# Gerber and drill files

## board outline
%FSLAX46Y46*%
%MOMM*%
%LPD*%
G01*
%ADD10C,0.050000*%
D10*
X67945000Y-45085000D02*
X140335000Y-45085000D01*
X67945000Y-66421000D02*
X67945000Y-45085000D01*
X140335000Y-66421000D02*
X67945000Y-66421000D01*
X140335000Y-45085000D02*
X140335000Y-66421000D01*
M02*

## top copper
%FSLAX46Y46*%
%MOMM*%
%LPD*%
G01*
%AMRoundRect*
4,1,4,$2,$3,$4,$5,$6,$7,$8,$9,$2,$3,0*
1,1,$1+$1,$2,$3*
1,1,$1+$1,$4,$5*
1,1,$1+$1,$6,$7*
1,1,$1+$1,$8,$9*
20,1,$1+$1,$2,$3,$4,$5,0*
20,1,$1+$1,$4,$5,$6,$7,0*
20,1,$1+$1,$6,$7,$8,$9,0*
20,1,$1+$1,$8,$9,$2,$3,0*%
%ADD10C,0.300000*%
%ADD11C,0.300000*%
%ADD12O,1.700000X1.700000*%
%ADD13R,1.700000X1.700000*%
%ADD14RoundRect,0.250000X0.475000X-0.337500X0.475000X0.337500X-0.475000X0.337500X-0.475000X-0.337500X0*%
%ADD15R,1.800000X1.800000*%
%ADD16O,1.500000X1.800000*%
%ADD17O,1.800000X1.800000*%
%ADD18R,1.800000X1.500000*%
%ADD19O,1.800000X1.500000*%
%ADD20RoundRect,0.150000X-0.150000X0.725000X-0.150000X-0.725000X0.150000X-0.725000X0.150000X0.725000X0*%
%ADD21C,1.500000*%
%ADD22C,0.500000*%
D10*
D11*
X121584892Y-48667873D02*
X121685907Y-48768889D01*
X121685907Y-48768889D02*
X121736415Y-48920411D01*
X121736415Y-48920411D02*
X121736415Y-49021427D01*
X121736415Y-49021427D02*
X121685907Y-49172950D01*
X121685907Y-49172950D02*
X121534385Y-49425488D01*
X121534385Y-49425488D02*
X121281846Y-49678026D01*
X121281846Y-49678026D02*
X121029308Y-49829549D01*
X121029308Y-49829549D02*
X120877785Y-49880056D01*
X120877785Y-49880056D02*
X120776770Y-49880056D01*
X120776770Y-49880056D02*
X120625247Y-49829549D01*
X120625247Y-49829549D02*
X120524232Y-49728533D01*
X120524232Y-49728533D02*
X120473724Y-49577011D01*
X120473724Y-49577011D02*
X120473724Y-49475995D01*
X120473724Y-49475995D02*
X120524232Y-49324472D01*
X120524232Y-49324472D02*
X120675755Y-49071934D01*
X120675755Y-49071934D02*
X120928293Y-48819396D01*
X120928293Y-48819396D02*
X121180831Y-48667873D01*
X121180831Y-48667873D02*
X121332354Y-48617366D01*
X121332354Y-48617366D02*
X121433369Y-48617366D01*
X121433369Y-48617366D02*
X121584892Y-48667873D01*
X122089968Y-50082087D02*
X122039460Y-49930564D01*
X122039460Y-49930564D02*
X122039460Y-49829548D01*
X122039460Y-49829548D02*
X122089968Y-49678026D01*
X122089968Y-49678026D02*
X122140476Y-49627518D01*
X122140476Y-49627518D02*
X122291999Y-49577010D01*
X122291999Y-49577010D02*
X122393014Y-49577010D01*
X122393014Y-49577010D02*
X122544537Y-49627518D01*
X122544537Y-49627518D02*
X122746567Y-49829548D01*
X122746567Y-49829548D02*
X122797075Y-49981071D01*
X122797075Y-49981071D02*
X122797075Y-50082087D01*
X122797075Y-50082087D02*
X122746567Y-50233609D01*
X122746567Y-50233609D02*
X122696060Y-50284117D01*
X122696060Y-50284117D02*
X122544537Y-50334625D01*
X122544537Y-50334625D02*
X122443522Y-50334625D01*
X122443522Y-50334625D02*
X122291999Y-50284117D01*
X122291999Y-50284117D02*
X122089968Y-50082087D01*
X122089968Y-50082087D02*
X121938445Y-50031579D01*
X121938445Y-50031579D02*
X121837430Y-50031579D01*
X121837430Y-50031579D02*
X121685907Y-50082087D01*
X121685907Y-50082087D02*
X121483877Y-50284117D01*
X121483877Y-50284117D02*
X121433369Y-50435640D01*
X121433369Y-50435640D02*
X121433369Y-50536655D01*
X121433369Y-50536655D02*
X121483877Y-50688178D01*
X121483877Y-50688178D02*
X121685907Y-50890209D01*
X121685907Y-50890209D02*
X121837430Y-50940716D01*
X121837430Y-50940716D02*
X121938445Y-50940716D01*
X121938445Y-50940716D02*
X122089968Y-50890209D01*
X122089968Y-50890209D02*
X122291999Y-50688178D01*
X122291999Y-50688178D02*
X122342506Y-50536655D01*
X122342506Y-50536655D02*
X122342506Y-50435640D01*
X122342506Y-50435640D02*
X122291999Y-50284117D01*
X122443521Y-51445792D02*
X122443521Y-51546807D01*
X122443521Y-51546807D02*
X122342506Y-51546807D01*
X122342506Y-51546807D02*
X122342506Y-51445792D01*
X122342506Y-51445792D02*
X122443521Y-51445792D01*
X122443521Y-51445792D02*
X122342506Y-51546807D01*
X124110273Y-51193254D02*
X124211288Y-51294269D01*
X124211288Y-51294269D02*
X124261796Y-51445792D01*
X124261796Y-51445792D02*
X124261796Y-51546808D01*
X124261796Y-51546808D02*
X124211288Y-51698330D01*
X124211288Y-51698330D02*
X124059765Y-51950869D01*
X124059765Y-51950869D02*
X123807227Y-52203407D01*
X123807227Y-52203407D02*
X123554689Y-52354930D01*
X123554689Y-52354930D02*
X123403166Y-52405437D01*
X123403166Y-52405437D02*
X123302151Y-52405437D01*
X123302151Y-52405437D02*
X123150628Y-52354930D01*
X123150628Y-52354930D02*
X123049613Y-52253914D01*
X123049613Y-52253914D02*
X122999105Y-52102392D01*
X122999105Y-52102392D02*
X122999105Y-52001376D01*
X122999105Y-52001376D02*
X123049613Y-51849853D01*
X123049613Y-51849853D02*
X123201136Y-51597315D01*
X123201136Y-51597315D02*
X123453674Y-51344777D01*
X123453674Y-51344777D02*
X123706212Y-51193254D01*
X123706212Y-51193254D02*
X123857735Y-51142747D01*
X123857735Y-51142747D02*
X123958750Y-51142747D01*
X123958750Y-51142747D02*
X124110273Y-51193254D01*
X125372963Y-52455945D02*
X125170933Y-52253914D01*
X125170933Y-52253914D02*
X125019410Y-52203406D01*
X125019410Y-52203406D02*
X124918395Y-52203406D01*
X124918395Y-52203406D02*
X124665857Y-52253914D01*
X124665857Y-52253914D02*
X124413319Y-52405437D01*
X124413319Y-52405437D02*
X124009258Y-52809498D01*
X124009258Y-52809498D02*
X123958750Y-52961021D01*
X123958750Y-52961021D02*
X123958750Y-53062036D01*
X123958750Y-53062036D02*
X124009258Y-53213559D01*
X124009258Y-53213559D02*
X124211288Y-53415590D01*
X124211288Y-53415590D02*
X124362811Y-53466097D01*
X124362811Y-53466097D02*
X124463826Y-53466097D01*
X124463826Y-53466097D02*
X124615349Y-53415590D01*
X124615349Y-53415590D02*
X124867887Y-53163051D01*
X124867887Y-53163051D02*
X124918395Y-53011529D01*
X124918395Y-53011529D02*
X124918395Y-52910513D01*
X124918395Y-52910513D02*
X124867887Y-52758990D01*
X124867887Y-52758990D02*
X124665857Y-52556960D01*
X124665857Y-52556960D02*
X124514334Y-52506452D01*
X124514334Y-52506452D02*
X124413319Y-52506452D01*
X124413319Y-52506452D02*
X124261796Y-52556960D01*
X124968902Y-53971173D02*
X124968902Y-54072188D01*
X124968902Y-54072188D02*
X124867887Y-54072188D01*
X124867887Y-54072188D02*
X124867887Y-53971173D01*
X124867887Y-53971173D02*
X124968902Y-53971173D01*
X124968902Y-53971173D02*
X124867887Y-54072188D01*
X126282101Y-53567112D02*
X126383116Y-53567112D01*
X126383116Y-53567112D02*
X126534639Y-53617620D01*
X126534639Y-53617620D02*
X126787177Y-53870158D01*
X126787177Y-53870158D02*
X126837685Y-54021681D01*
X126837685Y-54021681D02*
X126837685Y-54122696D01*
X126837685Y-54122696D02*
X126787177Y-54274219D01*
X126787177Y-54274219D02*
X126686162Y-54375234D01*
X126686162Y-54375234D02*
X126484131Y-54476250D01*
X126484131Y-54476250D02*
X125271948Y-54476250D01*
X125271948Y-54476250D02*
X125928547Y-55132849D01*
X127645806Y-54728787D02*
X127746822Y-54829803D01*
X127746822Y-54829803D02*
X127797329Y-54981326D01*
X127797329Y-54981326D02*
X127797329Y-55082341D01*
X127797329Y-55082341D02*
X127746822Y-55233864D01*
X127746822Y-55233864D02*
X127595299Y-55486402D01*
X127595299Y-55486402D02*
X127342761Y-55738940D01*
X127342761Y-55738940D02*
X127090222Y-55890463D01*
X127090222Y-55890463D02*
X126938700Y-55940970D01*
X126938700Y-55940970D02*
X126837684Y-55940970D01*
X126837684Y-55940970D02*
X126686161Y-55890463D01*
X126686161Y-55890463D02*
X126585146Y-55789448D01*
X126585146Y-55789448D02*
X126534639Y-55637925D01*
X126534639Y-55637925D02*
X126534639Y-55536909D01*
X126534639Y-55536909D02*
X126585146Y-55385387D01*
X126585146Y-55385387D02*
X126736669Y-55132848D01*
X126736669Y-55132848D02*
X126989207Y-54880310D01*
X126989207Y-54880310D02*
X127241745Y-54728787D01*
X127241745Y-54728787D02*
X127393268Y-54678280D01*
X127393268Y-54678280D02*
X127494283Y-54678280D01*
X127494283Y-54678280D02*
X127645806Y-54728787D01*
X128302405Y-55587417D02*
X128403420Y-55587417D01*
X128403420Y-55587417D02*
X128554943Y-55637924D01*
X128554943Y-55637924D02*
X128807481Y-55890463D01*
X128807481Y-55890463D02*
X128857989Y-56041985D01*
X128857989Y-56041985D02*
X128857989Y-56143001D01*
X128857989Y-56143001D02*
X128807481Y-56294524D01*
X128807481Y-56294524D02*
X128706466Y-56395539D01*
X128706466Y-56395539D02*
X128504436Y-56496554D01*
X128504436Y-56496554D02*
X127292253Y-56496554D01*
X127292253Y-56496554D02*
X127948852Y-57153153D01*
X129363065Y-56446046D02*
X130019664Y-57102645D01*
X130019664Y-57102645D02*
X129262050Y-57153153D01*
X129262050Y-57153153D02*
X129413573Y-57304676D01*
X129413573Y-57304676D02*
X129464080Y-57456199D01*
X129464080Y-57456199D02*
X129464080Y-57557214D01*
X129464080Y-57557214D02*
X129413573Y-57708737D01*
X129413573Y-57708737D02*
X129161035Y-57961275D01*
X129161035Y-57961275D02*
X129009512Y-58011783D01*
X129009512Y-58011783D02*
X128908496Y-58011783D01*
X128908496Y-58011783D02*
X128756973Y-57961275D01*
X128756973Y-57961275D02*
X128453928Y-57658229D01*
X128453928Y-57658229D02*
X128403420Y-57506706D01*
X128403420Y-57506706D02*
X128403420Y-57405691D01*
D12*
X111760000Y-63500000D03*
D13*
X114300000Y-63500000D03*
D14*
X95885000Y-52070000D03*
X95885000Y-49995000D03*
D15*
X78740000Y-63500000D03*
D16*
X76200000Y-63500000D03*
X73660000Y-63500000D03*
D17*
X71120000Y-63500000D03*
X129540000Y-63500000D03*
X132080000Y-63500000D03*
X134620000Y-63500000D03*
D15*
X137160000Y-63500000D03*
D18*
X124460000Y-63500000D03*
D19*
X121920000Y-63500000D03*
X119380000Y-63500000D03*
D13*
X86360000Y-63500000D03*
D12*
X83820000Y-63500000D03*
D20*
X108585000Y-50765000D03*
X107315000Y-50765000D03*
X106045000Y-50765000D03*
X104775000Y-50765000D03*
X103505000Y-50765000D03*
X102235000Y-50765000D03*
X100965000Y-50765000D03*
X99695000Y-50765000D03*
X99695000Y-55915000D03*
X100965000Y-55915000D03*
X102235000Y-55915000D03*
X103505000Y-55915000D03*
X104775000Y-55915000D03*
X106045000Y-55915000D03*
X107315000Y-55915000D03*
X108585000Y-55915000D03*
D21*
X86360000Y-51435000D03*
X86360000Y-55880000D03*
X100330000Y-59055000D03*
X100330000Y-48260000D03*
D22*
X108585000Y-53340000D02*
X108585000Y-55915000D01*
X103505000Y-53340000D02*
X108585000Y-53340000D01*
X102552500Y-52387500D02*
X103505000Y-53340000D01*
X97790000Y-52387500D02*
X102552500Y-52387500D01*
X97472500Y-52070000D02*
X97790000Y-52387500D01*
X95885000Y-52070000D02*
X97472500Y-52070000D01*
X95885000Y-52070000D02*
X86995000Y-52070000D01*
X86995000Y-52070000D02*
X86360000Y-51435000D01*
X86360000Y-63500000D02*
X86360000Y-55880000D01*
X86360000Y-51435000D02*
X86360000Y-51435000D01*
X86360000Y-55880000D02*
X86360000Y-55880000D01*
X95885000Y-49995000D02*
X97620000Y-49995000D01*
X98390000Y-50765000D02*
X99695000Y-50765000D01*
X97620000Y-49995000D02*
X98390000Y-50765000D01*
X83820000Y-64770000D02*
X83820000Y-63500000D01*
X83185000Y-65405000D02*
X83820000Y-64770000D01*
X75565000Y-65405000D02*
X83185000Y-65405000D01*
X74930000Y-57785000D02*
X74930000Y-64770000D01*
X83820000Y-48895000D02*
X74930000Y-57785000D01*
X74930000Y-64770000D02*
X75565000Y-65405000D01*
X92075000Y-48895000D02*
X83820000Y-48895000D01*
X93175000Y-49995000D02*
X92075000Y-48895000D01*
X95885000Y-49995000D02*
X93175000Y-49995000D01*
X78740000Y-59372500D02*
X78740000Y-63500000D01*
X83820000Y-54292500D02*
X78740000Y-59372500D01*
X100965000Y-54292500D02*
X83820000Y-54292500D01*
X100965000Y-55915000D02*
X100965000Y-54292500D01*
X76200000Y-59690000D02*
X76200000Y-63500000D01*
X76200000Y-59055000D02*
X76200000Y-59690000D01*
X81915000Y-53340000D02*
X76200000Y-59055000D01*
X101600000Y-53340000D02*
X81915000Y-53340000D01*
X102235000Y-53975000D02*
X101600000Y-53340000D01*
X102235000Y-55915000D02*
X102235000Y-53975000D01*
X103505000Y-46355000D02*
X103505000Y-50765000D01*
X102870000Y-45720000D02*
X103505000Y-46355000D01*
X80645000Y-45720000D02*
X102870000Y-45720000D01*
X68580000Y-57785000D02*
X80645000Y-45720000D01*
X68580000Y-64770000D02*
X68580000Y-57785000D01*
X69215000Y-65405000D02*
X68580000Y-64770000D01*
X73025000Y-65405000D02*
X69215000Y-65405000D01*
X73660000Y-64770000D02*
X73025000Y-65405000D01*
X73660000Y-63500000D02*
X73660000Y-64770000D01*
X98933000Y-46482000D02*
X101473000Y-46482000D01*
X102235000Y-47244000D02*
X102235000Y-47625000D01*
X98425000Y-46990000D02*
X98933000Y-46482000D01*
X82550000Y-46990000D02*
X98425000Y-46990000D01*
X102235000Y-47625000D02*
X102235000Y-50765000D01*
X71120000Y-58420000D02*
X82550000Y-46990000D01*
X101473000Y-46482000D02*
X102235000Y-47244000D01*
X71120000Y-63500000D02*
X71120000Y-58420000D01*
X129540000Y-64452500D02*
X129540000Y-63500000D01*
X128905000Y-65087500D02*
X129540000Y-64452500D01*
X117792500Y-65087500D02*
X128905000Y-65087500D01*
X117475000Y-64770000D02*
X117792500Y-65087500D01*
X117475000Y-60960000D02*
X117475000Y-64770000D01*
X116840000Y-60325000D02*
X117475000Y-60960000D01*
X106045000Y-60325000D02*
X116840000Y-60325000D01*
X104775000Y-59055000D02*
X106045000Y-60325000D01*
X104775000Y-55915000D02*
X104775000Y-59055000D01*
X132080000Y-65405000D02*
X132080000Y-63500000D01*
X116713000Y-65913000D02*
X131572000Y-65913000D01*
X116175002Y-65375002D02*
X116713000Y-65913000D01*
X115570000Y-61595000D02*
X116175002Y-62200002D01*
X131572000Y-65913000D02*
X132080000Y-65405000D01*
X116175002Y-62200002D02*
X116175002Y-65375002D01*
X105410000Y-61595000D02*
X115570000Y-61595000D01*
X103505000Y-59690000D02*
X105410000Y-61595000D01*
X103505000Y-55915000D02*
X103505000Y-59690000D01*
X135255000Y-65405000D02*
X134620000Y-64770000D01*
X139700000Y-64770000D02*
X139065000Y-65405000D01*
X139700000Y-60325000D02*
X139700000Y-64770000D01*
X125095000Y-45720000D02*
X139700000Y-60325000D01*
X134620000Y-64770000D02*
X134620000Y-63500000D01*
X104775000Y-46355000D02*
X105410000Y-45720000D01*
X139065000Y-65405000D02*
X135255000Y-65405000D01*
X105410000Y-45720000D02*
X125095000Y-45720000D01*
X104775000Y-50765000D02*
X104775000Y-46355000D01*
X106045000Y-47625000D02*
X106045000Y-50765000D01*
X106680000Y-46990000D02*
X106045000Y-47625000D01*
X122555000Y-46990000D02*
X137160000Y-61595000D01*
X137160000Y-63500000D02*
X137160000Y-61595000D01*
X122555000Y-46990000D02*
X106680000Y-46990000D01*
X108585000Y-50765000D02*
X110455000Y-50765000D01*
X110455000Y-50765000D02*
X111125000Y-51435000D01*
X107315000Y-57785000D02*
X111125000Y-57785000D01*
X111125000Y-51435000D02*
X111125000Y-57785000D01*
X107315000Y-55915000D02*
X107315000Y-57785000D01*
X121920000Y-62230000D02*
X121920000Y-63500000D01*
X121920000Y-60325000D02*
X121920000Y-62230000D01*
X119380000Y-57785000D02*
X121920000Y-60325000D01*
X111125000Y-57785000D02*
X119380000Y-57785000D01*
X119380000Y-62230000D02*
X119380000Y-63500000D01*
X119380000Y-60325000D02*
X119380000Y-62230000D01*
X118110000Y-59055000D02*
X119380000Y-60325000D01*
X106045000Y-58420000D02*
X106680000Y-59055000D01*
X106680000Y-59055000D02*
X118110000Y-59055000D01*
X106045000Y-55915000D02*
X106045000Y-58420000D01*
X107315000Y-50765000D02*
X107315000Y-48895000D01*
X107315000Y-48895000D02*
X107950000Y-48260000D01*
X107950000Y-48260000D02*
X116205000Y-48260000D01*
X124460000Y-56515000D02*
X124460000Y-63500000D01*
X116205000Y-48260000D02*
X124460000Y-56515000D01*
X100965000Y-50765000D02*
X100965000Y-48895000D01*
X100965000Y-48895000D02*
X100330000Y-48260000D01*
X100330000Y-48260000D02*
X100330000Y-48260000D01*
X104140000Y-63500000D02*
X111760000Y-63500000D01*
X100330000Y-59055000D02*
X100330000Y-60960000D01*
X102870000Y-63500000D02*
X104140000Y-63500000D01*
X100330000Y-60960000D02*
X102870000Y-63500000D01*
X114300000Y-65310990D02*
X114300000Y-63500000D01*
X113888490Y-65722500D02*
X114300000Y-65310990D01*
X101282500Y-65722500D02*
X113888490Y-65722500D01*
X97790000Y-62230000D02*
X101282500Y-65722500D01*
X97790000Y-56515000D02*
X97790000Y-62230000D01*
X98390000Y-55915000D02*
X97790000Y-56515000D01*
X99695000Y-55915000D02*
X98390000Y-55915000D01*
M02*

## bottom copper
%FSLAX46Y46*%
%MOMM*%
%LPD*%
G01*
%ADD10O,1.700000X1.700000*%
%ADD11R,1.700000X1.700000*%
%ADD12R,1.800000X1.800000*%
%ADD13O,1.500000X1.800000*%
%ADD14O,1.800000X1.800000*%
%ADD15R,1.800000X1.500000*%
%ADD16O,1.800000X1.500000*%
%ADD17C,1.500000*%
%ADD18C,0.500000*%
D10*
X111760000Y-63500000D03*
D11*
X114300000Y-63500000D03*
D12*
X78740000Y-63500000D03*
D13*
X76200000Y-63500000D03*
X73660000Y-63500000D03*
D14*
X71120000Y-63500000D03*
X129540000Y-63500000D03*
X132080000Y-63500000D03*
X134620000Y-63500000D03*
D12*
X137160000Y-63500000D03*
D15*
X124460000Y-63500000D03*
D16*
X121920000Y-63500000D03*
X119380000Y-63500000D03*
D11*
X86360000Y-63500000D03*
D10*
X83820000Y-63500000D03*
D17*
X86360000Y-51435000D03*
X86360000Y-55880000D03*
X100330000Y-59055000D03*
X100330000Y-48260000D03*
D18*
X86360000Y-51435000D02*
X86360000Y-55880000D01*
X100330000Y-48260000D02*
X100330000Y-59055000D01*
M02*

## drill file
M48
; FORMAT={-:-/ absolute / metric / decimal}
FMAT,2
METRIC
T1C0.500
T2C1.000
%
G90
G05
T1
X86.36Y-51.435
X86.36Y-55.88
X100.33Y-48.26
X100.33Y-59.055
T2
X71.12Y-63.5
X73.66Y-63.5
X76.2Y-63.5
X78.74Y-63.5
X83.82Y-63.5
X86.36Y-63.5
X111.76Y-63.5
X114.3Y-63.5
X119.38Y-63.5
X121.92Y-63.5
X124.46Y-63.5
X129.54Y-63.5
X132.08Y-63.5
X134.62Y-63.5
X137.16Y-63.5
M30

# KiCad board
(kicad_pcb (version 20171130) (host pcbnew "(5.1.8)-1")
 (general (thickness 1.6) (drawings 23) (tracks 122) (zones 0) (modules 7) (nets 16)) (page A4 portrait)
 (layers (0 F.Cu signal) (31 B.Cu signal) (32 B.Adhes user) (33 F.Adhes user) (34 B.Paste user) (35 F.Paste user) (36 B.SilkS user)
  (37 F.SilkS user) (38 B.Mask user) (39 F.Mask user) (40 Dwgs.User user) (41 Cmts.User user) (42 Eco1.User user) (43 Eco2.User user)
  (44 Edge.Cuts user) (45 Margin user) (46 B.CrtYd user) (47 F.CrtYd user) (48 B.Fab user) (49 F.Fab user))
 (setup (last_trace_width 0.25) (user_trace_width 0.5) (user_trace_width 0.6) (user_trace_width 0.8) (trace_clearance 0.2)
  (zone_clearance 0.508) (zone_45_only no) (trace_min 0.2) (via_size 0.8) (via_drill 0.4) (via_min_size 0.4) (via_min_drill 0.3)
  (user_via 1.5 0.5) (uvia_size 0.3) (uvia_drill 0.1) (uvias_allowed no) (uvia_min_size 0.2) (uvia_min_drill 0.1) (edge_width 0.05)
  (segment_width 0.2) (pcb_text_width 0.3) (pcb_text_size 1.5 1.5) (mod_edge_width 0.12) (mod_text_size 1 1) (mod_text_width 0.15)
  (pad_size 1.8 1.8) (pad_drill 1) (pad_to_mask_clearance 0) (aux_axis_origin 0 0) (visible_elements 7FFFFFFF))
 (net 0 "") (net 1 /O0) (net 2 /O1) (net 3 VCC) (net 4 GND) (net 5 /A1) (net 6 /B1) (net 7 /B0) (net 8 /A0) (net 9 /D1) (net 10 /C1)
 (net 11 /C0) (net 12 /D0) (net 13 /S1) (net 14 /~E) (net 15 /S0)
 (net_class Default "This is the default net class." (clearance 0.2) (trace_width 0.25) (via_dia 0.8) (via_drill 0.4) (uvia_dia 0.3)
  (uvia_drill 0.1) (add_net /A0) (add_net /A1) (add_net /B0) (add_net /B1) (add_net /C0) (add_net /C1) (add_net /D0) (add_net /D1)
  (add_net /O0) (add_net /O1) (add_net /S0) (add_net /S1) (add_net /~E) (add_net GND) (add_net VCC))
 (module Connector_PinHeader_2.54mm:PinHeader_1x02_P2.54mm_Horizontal (layer F.Cu) (at 114.3 63.5 270)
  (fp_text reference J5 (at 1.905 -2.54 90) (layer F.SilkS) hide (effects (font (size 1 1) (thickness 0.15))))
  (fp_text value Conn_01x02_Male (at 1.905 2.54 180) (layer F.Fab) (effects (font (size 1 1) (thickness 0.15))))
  (pad 2 thru_hole oval (at 0 2.54 270) (size 1.7 1.7) (drill 1) (layers *.Cu *.Mask) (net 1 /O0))
  (pad 1 thru_hole rect (at 0 0 270) (size 1.7 1.7) (drill 1) (layers *.Cu *.Mask) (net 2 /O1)))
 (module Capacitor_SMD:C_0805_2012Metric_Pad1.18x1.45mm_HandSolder (layer F.Cu) (at 95.885 51.0325 90)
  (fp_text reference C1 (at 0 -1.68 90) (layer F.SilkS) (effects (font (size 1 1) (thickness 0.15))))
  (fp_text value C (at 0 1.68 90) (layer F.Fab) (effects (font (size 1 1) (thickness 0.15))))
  (pad 1 smd roundrect (at -1.0375 0 90) (size 1.175 1.45) (layers F.Cu F.Paste F.Mask) (roundrect_rratio 0.2127659574468085) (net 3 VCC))
  (pad 2 smd roundrect (at 1.0375 0 90) (size 1.175 1.45) (layers F.Cu F.Paste F.Mask) (roundrect_rratio 0.2127659574468085) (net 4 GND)))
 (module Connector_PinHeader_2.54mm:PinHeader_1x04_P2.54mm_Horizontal (layer F.Cu) (at 78.74 63.5 270)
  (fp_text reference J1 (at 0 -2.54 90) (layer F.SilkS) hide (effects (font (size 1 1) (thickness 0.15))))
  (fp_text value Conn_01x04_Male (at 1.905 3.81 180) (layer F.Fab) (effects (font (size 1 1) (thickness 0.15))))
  (pad 1 thru_hole rect (at 0 0 270) (size 1.8 1.8) (drill 1) (layers *.Cu *.Mask) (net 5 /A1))
  (pad 2 thru_hole oval (at 0 2.54 270) (size 1.8 1.5) (drill 1) (layers *.Cu *.Mask) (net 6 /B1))
  (pad 3 thru_hole oval (at 0 5.08 270) (size 1.8 1.5) (drill 1) (layers *.Cu *.Mask) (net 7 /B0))
  (pad 4 thru_hole oval (at 0 7.62 270) (size 1.8 1.8) (drill 1) (layers *.Cu *.Mask) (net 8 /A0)))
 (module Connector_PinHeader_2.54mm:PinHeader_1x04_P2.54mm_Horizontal (layer F.Cu) (at 137.16 63.5 270)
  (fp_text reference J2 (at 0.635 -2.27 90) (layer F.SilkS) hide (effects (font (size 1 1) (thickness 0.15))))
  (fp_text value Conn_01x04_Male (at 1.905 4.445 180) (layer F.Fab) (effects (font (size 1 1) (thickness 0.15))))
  (pad 4 thru_hole oval (at 0 7.62 270) (size 1.8 1.8) (drill 1) (layers *.Cu *.Mask) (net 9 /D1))
  (pad 3 thru_hole oval (at 0 5.08 270) (size 1.8 1.8) (drill 1) (layers *.Cu *.Mask) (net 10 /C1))
  (pad 2 thru_hole oval (at 0 2.54 270) (size 1.8 1.8) (drill 1) (layers *.Cu *.Mask) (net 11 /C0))
  (pad 1 thru_hole rect (at 0 0 270) (size 1.8 1.8) (drill 1) (layers *.Cu *.Mask) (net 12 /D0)))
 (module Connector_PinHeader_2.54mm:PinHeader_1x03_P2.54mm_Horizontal (layer F.Cu) (at 124.46 63.5 270)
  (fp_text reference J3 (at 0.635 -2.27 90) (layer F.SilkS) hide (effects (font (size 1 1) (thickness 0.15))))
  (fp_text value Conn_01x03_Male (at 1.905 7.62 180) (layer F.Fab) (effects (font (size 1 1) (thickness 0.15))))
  (pad 1 thru_hole rect (at 0 0 270) (size 1.5 1.8) (drill 1) (layers *.Cu *.Mask) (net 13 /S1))
  (pad 2 thru_hole oval (at 0 2.54 270) (size 1.5 1.8) (drill 1) (layers *.Cu *.Mask) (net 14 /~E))
  (pad 3 thru_hole oval (at 0 5.08 270) (size 1.5 1.8) (drill 1) (layers *.Cu *.Mask) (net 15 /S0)))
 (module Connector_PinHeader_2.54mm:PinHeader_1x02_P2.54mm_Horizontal (layer F.Cu) (at 86.36 63.5 270)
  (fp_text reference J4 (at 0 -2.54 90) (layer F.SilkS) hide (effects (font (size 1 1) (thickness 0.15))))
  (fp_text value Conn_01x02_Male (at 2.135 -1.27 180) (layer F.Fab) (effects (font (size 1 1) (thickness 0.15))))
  (pad 1 thru_hole rect (at 0 0 270) (size 1.7 1.7) (drill 1) (layers *.Cu *.Mask) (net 3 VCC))
  (pad 2 thru_hole oval (at 0 2.54 270) (size 1.7 1.7) (drill 1) (layers *.Cu *.Mask) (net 4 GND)))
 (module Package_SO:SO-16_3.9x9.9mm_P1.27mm (layer F.Cu) (at 104.14 53.34 270)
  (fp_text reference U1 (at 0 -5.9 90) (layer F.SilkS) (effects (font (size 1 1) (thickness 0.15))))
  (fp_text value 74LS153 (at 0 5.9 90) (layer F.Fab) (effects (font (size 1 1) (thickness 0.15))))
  (pad 1 smd roundrect (at -2.575 -4.445 270) (size 1.75 0.6) (layers F.Cu F.Paste F.Mask) (roundrect_rratio 0.25) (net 14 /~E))
  (pad 2 smd roundrect (at -2.575 -3.175 270) (size 1.75 0.6) (layers F.Cu F.Paste F.Mask) (roundrect_rratio 0.25) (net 13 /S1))
  (pad 3 smd roundrect (at -2.575 -1.905 270) (size 1.75 0.6) (layers F.Cu F.Paste F.Mask) (roundrect_rratio 0.25) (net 12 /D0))
  (pad 4 smd roundrect (at -2.575 -0.635 270) (size 1.75 0.6) (layers F.Cu F.Paste F.Mask) (roundrect_rratio 0.25) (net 11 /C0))
  (pad 5 smd roundrect (at -2.575 0.635 270) (size 1.75 0.6) (layers F.Cu F.Paste F.Mask) (roundrect_rratio 0.25) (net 7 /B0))
  (pad 6 smd roundrect (at -2.575 1.905 270) (size 1.75 0.6) (layers F.Cu F.Paste F.Mask) (roundrect_rratio 0.25) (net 8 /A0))
  (pad 7 smd roundrect (at -2.575 3.175 270) (size 1.75 0.6) (layers F.Cu F.Paste F.Mask) (roundrect_rratio 0.25) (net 1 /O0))
  (pad 8 smd roundrect (at -2.575 4.445 270) (size 1.75 0.6) (layers F.Cu F.Paste F.Mask) (roundrect_rratio 0.25) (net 4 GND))
  (pad 9 smd roundrect (at 2.575 4.445 270) (size 1.75 0.6) (layers F.Cu F.Paste F.Mask) (roundrect_rratio 0.25) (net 2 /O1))
  (pad 10 smd roundrect (at 2.575 3.175 270) (size 1.75 0.6) (layers F.Cu F.Paste F.Mask) (roundrect_rratio 0.25) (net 5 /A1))
  (pad 11 smd roundrect (at 2.575 1.905 270) (size 1.75 0.6) (layers F.Cu F.Paste F.Mask) (roundrect_rratio 0.25) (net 6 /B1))
  (pad 12 smd roundrect (at 2.575 0.635 270) (size 1.75 0.6) (layers F.Cu F.Paste F.Mask) (roundrect_rratio 0.25) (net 10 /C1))
  (pad 13 smd roundrect (at 2.575 -0.635 270) (size 1.75 0.6) (layers F.Cu F.Paste F.Mask) (roundrect_rratio 0.25) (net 9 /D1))
  (pad 14 smd roundrect (at 2.575 -1.905 270) (size 1.75 0.6) (layers F.Cu F.Paste F.Mask) (roundrect_rratio 0.25) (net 15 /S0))
  (pad 15 smd roundrect (at 2.575 -3.175 270) (size 1.75 0.6) (layers F.Cu F.Paste F.Mask) (roundrect_rratio 0.25) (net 14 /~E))
  (pad 16 smd roundrect (at 2.575 -4.445 270) (size 1.75 0.6) (layers F.Cu F.Paste F.Mask) (roundrect_rratio 0.25) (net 3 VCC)))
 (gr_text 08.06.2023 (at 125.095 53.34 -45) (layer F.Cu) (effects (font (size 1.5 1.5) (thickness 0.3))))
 (gr_line (start 67.945 45.085) (end 140.335 45.085) (layer Edge.Cuts) (width 0.05))
 (gr_line (start 67.945 66.421) (end 67.945 45.085) (layer Edge.Cuts) (width 0.05))
 (gr_line (start 140.335 66.421) (end 67.945 66.421) (layer Edge.Cuts) (width 0.05))
 (gr_line (start 140.335 45.085) (end 140.335 66.421) (layer Edge.Cuts) (width 0.05))
 (segment (start 108.585 53.34) (end 108.585 55.915) (width 0.5) (layer F.Cu) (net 3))
 (segment (start 103.505 53.34) (end 108.585 53.34) (width 0.5) (layer F.Cu) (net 3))
 (segment (start 102.5525 52.3875) (end 103.505 53.34) (width 0.5) (layer F.Cu) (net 3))
 (segment (start 97.79 52.3875) (end 102.5525 52.3875) (width 0.5) (layer F.Cu) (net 3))
 (segment (start 97.4725 52.07) (end 97.79 52.3875) (width 0.5) (layer F.Cu) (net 3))
 (segment (start 95.885 52.07) (end 97.4725 52.07) (width 0.5) (layer F.Cu) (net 3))
 (segment (start 95.885 52.07) (end 86.995 52.07) (width 0.5) (layer F.Cu) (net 3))
 (segment (start 86.995 52.07) (end 86.36 51.435) (width 0.5) (layer F.Cu) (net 3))
 (segment (start 86.36 63.5) (end 86.36 55.88) (width 0.5) (layer F.Cu) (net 3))
 (segment (start 86.36 51.435) (end 86.36 51.435) (width 0.5) (layer F.Cu) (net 3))
 (via (at 86.36 51.435) (size 1.5) (drill 0.5) (layers F.Cu B.Cu) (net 3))
 (segment (start 86.36 55.88) (end 86.36 55.88) (width 0.5) (layer F.Cu) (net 3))
 (via (at 86.36 55.88) (size 1.5) (drill 0.5) (layers F.Cu B.Cu) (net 3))
 (segment (start 86.36 51.435) (end 86.36 55.88) (width 0.5) (layer B.Cu) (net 3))
 (segment (start 95.885 49.995) (end 97.62 49.995) (width 0.5) (layer F.Cu) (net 4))
 (segment (start 98.39 50.765) (end 99.695 50.765) (width 0.5) (layer F.Cu) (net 4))
 (segment (start 97.62 49.995) (end 98.39 50.765) (width 0.5) (layer F.Cu) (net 4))
 (segment (start 83.82 64.77) (end 83.82 63.5) (width 0.5) (layer F.Cu) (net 4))
 (segment (start 83.185 65.405) (end 83.82 64.77) (width 0.5) (layer F.Cu) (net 4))
 (segment (start 75.565 65.405) (end 83.185 65.405) (width 0.5) (layer F.Cu) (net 4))
 (segment (start 74.93 57.785) (end 74.93 64.77) (width 0.5) (layer F.Cu) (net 4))
 (segment (start 83.82 48.895) (end 74.93 57.785) (width 0.5) (layer F.Cu) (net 4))
 (segment (start 74.93 64.77) (end 75.565 65.405) (width 0.5) (layer F.Cu) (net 4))
 (segment (start 92.075 48.895) (end 83.82 48.895) (width 0.5) (layer F.Cu) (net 4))
 (segment (start 93.175 49.995) (end 92.075 48.895) (width 0.5) (layer F.Cu) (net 4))
 (segment (start 95.885 49.995) (end 93.175 49.995) (width 0.5) (layer F.Cu) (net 4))
 (segment (start 78.74 59.3725) (end 78.74 63.5) (width 0.5) (layer F.Cu) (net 5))
 (segment (start 83.82 54.2925) (end 78.74 59.3725) (width 0.5) (layer F.Cu) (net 5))
 (segment (start 100.965 54.2925) (end 83.82 54.2925) (width 0.5) (layer F.Cu) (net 5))
 (segment (start 100.965 55.915) (end 100.965 54.2925) (width 0.5) (layer F.Cu) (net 5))
 (segment (start 76.2 59.69) (end 76.2 63.5) (width 0.5) (layer F.Cu) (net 6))
 (segment (start 76.2 59.055) (end 76.2 59.69) (width 0.5) (layer F.Cu) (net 6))
 (segment (start 81.915 53.34) (end 76.2 59.055) (width 0.5) (layer F.Cu) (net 6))
 (segment (start 101.6 53.34) (end 81.915 53.34) (width 0.5) (layer F.Cu) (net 6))
 (segment (start 102.235 53.975) (end 101.6 53.34) (width 0.5) (layer F.Cu) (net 6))
 (segment (start 102.235 55.915) (end 102.235 53.975) (width 0.5) (layer F.Cu) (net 6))
 (segment (start 103.505 46.355) (end 103.505 50.765) (width 0.5) (layer F.Cu) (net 7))
 (segment (start 102.87 45.72) (end 103.505 46.355) (width 0.5) (layer F.Cu) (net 7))
 (segment (start 80.645 45.72) (end 102.87 45.72) (width 0.5) (layer F.Cu) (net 7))
 (segment (start 68.58 57.785) (end 80.645 45.72) (width 0.5) (layer F.Cu) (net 7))
 (segment (start 68.58 64.77) (end 68.58 57.785) (width 0.5) (layer F.Cu) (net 7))
 (segment (start 69.215 65.405) (end 68.58 64.77) (width 0.5) (layer F.Cu) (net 7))
 (segment (start 73.025 65.405) (end 69.215 65.405) (width 0.5) (layer F.Cu) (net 7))
 (segment (start 73.66 64.77) (end 73.025 65.405) (width 0.5) (layer F.Cu) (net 7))
 (segment (start 73.66 63.5) (end 73.66 64.77) (width 0.5) (layer F.Cu) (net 7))
 (segment (start 98.933 46.482) (end 101.473 46.482) (width 0.5) (layer F.Cu) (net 8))
 (segment (start 102.235 47.244) (end 102.235 47.625) (width 0.5) (layer F.Cu) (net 8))
 (segment (start 98.425 46.99) (end 98.933 46.482) (width 0.5) (layer F.Cu) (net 8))
 (segment (start 82.55 46.99) (end 98.425 46.99) (width 0.5) (layer F.Cu) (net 8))
 (segment (start 102.235 47.625) (end 102.235 50.765) (width 0.5) (layer F.Cu) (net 8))
 (segment (start 71.12 58.42) (end 82.55 46.99) (width 0.5) (layer F.Cu) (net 8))
 (segment (start 101.473 46.482) (end 102.235 47.244) (width 0.5) (layer F.Cu) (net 8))
 (segment (start 71.12 63.5) (end 71.12 58.42) (width 0.5) (layer F.Cu) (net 8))
 (segment (start 129.54 64.4525) (end 129.54 63.5) (width 0.5) (layer F.Cu) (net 9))
 (segment (start 128.905 65.0875) (end 129.54 64.4525) (width 0.5) (layer F.Cu) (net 9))
 (segment (start 117.7925 65.0875) (end 128.905 65.0875) (width 0.5) (layer F.Cu) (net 9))
 (segment (start 117.475 64.77) (end 117.7925 65.0875) (width 0.5) (layer F.Cu) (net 9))
 (segment (start 117.475 60.96) (end 117.475 64.77) (width 0.5) (layer F.Cu) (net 9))
 (segment (start 116.84 60.325) (end 117.475 60.96) (width 0.5) (layer F.Cu) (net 9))
 (segment (start 106.045 60.325) (end 116.84 60.325) (width 0.5) (layer F.Cu) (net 9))
 (segment (start 104.775 59.055) (end 106.045 60.325) (width 0.5) (layer F.Cu) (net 9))
 (segment (start 104.775 55.915) (end 104.775 59.055) (width 0.5) (layer F.Cu) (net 9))
 (segment (start 132.08 65.405) (end 132.08 63.5) (width 0.5) (layer F.Cu) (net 10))
 (segment (start 116.713 65.913) (end 131.572 65.913) (width 0.5) (layer F.Cu) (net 10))
 (segment (start 116.175002 65.375002) (end 116.713 65.913) (width 0.5) (layer F.Cu) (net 10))
 (segment (start 115.57 61.595) (end 116.175002 62.200002) (width 0.5) (layer F.Cu) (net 10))
 (segment (start 131.572 65.913) (end 132.08 65.405) (width 0.5) (layer F.Cu) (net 10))
 (segment (start 116.175002 62.200002) (end 116.175002 65.375002) (width 0.5) (layer F.Cu) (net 10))
 (segment (start 105.41 61.595) (end 115.57 61.595) (width 0.5) (layer F.Cu) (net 10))
 (segment (start 103.505 59.69) (end 105.41 61.595) (width 0.5) (layer F.Cu) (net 10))
 (segment (start 103.505 55.915) (end 103.505 59.69) (width 0.5) (layer F.Cu) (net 10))
 (segment (start 135.255 65.405) (end 134.62 64.77) (width 0.5) (layer F.Cu) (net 11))
 (segment (start 139.7 64.77) (end 139.065 65.405) (width 0.5) (layer F.Cu) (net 11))
 (segment (start 139.7 60.325) (end 139.7 64.77) (width 0.5) (layer F.Cu) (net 11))
 (segment (start 125.095 45.72) (end 139.7 60.325) (width 0.5) (layer F.Cu) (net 11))
 (segment (start 134.62 64.77) (end 134.62 63.5) (width 0.5) (layer F.Cu) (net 11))
 (segment (start 104.775 46.355) (end 105.41 45.72) (width 0.5) (layer F.Cu) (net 11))
 (segment (start 139.065 65.405) (end 135.255 65.405) (width 0.5) (layer F.Cu) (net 11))
 (segment (start 105.41 45.72) (end 125.095 45.72) (width 0.5) (layer F.Cu) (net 11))
 (segment (start 104.775 50.765) (end 104.775 46.355) (width 0.5) (layer F.Cu) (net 11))
 (segment (start 106.045 47.625) (end 106.045 50.765) (width 0.5) (layer F.Cu) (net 12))
 (segment (start 106.68 46.99) (end 106.045 47.625) (width 0.5) (layer F.Cu) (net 12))
 (segment (start 122.555 46.99) (end 137.16 61.595) (width 0.5) (layer F.Cu) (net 12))
 (segment (start 137.16 63.5) (end 137.16 61.595) (width 0.5) (layer F.Cu) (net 12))
 (segment (start 122.555 46.99) (end 106.68 46.99) (width 0.5) (layer F.Cu) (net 12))
 (segment (start 108.585 50.765) (end 110.455 50.765) (width 0.5) (layer F.Cu) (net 14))
 (segment (start 110.455 50.765) (end 111.125 51.435) (width 0.5) (layer F.Cu) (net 14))
 (segment (start 107.315 57.785) (end 111.125 57.785) (width 0.5) (layer F.Cu) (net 14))
 (segment (start 111.125 51.435) (end 111.125 57.785) (width 0.5) (layer F.Cu) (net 14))
 (segment (start 107.315 55.915) (end 107.315 57.785) (width 0.5) (layer F.Cu) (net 14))
 (segment (start 121.92 62.23) (end 121.92 63.5) (width 0.5) (layer F.Cu) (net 14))
 (segment (start 121.92 60.325) (end 121.92 62.23) (width 0.5) (layer F.Cu) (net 14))
 (segment (start 119.38 57.785) (end 121.92 60.325) (width 0.5) (layer F.Cu) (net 14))
 (segment (start 111.125 57.785) (end 119.38 57.785) (width 0.5) (layer F.Cu) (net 14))
 (segment (start 119.38 62.23) (end 119.38 63.5) (width 0.5) (layer F.Cu) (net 15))
 (segment (start 119.38 60.325) (end 119.38 62.23) (width 0.5) (layer F.Cu) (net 15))
 (segment (start 118.11 59.055) (end 119.38 60.325) (width 0.5) (layer F.Cu) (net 15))
 (segment (start 106.045 58.42) (end 106.68 59.055) (width 0.5) (layer F.Cu) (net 15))
 (segment (start 106.68 59.055) (end 118.11 59.055) (width 0.5) (layer F.Cu) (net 15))
 (segment (start 106.045 55.915) (end 106.045 58.42) (width 0.5) (layer F.Cu) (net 15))
 (segment (start 107.315 50.765) (end 107.315 48.895) (width 0.5) (layer F.Cu) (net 13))
 (segment (start 107.315 48.895) (end 107.95 48.26) (width 0.5) (layer F.Cu) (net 13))
 (segment (start 107.95 48.26) (end 116.205 48.26) (width 0.5) (layer F.Cu) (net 13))
 (segment (start 124.46 56.515) (end 124.46 63.5) (width 0.5) (layer F.Cu) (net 13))
 (segment (start 116.205 48.26) (end 124.46 56.515) (width 0.5) (layer F.Cu) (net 13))
 (via (at 100.33 59.055) (size 1.5) (drill 0.5) (layers F.Cu B.Cu) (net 1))
 (segment (start 100.965 50.765) (end 100.965 48.895) (width 0.5) (layer F.Cu) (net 1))
 (segment (start 100.965 48.895) (end 100.33 48.26) (width 0.5) (layer F.Cu) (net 1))
 (segment (start 100.33 48.26) (end 100.33 48.26) (width 0.5) (layer F.Cu) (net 1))
 (via (at 100.33 48.26) (size 1.5) (drill 0.5) (layers F.Cu B.Cu) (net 1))
 (segment (start 100.33 48.26) (end 100.33 59.055) (width 0.5) (layer B.Cu) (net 1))
 (segment (start 104.14 63.5) (end 111.76 63.5) (width 0.5) (layer F.Cu) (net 1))
 (segment (start 100.33 59.055) (end 100.33 60.96) (width 0.5) (layer F.Cu) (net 1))
 (segment (start 102.87 63.5) (end 104.14 63.5) (width 0.5) (layer F.Cu) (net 1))
 (segment (start 100.33 60.96) (end 102.87 63.5) (width 0.5) (layer F.Cu) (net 1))
 (segment (start 114.3 65.31099) (end 114.3 63.5) (width 0.5) (layer F.Cu) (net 2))
 (segment (start 113.88849 65.7225) (end 114.3 65.31099) (width 0.5) (layer F.Cu) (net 2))
 (segment (start 101.2825 65.7225) (end 113.88849 65.7225) (width 0.5) (layer F.Cu) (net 2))
 (segment (start 97.79 62.23) (end 101.2825 65.7225) (width 0.5) (layer F.Cu) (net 2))
 (segment (start 97.79 56.515) (end 97.79 62.23) (width 0.5) (layer F.Cu) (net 2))
 (segment (start 98.39 55.915) (end 97.79 56.515) (width 0.5) (layer F.Cu) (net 2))
 (segment (start 99.695 55.915) (end 98.39 55.915) (width 0.5) (layer F.Cu) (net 2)))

